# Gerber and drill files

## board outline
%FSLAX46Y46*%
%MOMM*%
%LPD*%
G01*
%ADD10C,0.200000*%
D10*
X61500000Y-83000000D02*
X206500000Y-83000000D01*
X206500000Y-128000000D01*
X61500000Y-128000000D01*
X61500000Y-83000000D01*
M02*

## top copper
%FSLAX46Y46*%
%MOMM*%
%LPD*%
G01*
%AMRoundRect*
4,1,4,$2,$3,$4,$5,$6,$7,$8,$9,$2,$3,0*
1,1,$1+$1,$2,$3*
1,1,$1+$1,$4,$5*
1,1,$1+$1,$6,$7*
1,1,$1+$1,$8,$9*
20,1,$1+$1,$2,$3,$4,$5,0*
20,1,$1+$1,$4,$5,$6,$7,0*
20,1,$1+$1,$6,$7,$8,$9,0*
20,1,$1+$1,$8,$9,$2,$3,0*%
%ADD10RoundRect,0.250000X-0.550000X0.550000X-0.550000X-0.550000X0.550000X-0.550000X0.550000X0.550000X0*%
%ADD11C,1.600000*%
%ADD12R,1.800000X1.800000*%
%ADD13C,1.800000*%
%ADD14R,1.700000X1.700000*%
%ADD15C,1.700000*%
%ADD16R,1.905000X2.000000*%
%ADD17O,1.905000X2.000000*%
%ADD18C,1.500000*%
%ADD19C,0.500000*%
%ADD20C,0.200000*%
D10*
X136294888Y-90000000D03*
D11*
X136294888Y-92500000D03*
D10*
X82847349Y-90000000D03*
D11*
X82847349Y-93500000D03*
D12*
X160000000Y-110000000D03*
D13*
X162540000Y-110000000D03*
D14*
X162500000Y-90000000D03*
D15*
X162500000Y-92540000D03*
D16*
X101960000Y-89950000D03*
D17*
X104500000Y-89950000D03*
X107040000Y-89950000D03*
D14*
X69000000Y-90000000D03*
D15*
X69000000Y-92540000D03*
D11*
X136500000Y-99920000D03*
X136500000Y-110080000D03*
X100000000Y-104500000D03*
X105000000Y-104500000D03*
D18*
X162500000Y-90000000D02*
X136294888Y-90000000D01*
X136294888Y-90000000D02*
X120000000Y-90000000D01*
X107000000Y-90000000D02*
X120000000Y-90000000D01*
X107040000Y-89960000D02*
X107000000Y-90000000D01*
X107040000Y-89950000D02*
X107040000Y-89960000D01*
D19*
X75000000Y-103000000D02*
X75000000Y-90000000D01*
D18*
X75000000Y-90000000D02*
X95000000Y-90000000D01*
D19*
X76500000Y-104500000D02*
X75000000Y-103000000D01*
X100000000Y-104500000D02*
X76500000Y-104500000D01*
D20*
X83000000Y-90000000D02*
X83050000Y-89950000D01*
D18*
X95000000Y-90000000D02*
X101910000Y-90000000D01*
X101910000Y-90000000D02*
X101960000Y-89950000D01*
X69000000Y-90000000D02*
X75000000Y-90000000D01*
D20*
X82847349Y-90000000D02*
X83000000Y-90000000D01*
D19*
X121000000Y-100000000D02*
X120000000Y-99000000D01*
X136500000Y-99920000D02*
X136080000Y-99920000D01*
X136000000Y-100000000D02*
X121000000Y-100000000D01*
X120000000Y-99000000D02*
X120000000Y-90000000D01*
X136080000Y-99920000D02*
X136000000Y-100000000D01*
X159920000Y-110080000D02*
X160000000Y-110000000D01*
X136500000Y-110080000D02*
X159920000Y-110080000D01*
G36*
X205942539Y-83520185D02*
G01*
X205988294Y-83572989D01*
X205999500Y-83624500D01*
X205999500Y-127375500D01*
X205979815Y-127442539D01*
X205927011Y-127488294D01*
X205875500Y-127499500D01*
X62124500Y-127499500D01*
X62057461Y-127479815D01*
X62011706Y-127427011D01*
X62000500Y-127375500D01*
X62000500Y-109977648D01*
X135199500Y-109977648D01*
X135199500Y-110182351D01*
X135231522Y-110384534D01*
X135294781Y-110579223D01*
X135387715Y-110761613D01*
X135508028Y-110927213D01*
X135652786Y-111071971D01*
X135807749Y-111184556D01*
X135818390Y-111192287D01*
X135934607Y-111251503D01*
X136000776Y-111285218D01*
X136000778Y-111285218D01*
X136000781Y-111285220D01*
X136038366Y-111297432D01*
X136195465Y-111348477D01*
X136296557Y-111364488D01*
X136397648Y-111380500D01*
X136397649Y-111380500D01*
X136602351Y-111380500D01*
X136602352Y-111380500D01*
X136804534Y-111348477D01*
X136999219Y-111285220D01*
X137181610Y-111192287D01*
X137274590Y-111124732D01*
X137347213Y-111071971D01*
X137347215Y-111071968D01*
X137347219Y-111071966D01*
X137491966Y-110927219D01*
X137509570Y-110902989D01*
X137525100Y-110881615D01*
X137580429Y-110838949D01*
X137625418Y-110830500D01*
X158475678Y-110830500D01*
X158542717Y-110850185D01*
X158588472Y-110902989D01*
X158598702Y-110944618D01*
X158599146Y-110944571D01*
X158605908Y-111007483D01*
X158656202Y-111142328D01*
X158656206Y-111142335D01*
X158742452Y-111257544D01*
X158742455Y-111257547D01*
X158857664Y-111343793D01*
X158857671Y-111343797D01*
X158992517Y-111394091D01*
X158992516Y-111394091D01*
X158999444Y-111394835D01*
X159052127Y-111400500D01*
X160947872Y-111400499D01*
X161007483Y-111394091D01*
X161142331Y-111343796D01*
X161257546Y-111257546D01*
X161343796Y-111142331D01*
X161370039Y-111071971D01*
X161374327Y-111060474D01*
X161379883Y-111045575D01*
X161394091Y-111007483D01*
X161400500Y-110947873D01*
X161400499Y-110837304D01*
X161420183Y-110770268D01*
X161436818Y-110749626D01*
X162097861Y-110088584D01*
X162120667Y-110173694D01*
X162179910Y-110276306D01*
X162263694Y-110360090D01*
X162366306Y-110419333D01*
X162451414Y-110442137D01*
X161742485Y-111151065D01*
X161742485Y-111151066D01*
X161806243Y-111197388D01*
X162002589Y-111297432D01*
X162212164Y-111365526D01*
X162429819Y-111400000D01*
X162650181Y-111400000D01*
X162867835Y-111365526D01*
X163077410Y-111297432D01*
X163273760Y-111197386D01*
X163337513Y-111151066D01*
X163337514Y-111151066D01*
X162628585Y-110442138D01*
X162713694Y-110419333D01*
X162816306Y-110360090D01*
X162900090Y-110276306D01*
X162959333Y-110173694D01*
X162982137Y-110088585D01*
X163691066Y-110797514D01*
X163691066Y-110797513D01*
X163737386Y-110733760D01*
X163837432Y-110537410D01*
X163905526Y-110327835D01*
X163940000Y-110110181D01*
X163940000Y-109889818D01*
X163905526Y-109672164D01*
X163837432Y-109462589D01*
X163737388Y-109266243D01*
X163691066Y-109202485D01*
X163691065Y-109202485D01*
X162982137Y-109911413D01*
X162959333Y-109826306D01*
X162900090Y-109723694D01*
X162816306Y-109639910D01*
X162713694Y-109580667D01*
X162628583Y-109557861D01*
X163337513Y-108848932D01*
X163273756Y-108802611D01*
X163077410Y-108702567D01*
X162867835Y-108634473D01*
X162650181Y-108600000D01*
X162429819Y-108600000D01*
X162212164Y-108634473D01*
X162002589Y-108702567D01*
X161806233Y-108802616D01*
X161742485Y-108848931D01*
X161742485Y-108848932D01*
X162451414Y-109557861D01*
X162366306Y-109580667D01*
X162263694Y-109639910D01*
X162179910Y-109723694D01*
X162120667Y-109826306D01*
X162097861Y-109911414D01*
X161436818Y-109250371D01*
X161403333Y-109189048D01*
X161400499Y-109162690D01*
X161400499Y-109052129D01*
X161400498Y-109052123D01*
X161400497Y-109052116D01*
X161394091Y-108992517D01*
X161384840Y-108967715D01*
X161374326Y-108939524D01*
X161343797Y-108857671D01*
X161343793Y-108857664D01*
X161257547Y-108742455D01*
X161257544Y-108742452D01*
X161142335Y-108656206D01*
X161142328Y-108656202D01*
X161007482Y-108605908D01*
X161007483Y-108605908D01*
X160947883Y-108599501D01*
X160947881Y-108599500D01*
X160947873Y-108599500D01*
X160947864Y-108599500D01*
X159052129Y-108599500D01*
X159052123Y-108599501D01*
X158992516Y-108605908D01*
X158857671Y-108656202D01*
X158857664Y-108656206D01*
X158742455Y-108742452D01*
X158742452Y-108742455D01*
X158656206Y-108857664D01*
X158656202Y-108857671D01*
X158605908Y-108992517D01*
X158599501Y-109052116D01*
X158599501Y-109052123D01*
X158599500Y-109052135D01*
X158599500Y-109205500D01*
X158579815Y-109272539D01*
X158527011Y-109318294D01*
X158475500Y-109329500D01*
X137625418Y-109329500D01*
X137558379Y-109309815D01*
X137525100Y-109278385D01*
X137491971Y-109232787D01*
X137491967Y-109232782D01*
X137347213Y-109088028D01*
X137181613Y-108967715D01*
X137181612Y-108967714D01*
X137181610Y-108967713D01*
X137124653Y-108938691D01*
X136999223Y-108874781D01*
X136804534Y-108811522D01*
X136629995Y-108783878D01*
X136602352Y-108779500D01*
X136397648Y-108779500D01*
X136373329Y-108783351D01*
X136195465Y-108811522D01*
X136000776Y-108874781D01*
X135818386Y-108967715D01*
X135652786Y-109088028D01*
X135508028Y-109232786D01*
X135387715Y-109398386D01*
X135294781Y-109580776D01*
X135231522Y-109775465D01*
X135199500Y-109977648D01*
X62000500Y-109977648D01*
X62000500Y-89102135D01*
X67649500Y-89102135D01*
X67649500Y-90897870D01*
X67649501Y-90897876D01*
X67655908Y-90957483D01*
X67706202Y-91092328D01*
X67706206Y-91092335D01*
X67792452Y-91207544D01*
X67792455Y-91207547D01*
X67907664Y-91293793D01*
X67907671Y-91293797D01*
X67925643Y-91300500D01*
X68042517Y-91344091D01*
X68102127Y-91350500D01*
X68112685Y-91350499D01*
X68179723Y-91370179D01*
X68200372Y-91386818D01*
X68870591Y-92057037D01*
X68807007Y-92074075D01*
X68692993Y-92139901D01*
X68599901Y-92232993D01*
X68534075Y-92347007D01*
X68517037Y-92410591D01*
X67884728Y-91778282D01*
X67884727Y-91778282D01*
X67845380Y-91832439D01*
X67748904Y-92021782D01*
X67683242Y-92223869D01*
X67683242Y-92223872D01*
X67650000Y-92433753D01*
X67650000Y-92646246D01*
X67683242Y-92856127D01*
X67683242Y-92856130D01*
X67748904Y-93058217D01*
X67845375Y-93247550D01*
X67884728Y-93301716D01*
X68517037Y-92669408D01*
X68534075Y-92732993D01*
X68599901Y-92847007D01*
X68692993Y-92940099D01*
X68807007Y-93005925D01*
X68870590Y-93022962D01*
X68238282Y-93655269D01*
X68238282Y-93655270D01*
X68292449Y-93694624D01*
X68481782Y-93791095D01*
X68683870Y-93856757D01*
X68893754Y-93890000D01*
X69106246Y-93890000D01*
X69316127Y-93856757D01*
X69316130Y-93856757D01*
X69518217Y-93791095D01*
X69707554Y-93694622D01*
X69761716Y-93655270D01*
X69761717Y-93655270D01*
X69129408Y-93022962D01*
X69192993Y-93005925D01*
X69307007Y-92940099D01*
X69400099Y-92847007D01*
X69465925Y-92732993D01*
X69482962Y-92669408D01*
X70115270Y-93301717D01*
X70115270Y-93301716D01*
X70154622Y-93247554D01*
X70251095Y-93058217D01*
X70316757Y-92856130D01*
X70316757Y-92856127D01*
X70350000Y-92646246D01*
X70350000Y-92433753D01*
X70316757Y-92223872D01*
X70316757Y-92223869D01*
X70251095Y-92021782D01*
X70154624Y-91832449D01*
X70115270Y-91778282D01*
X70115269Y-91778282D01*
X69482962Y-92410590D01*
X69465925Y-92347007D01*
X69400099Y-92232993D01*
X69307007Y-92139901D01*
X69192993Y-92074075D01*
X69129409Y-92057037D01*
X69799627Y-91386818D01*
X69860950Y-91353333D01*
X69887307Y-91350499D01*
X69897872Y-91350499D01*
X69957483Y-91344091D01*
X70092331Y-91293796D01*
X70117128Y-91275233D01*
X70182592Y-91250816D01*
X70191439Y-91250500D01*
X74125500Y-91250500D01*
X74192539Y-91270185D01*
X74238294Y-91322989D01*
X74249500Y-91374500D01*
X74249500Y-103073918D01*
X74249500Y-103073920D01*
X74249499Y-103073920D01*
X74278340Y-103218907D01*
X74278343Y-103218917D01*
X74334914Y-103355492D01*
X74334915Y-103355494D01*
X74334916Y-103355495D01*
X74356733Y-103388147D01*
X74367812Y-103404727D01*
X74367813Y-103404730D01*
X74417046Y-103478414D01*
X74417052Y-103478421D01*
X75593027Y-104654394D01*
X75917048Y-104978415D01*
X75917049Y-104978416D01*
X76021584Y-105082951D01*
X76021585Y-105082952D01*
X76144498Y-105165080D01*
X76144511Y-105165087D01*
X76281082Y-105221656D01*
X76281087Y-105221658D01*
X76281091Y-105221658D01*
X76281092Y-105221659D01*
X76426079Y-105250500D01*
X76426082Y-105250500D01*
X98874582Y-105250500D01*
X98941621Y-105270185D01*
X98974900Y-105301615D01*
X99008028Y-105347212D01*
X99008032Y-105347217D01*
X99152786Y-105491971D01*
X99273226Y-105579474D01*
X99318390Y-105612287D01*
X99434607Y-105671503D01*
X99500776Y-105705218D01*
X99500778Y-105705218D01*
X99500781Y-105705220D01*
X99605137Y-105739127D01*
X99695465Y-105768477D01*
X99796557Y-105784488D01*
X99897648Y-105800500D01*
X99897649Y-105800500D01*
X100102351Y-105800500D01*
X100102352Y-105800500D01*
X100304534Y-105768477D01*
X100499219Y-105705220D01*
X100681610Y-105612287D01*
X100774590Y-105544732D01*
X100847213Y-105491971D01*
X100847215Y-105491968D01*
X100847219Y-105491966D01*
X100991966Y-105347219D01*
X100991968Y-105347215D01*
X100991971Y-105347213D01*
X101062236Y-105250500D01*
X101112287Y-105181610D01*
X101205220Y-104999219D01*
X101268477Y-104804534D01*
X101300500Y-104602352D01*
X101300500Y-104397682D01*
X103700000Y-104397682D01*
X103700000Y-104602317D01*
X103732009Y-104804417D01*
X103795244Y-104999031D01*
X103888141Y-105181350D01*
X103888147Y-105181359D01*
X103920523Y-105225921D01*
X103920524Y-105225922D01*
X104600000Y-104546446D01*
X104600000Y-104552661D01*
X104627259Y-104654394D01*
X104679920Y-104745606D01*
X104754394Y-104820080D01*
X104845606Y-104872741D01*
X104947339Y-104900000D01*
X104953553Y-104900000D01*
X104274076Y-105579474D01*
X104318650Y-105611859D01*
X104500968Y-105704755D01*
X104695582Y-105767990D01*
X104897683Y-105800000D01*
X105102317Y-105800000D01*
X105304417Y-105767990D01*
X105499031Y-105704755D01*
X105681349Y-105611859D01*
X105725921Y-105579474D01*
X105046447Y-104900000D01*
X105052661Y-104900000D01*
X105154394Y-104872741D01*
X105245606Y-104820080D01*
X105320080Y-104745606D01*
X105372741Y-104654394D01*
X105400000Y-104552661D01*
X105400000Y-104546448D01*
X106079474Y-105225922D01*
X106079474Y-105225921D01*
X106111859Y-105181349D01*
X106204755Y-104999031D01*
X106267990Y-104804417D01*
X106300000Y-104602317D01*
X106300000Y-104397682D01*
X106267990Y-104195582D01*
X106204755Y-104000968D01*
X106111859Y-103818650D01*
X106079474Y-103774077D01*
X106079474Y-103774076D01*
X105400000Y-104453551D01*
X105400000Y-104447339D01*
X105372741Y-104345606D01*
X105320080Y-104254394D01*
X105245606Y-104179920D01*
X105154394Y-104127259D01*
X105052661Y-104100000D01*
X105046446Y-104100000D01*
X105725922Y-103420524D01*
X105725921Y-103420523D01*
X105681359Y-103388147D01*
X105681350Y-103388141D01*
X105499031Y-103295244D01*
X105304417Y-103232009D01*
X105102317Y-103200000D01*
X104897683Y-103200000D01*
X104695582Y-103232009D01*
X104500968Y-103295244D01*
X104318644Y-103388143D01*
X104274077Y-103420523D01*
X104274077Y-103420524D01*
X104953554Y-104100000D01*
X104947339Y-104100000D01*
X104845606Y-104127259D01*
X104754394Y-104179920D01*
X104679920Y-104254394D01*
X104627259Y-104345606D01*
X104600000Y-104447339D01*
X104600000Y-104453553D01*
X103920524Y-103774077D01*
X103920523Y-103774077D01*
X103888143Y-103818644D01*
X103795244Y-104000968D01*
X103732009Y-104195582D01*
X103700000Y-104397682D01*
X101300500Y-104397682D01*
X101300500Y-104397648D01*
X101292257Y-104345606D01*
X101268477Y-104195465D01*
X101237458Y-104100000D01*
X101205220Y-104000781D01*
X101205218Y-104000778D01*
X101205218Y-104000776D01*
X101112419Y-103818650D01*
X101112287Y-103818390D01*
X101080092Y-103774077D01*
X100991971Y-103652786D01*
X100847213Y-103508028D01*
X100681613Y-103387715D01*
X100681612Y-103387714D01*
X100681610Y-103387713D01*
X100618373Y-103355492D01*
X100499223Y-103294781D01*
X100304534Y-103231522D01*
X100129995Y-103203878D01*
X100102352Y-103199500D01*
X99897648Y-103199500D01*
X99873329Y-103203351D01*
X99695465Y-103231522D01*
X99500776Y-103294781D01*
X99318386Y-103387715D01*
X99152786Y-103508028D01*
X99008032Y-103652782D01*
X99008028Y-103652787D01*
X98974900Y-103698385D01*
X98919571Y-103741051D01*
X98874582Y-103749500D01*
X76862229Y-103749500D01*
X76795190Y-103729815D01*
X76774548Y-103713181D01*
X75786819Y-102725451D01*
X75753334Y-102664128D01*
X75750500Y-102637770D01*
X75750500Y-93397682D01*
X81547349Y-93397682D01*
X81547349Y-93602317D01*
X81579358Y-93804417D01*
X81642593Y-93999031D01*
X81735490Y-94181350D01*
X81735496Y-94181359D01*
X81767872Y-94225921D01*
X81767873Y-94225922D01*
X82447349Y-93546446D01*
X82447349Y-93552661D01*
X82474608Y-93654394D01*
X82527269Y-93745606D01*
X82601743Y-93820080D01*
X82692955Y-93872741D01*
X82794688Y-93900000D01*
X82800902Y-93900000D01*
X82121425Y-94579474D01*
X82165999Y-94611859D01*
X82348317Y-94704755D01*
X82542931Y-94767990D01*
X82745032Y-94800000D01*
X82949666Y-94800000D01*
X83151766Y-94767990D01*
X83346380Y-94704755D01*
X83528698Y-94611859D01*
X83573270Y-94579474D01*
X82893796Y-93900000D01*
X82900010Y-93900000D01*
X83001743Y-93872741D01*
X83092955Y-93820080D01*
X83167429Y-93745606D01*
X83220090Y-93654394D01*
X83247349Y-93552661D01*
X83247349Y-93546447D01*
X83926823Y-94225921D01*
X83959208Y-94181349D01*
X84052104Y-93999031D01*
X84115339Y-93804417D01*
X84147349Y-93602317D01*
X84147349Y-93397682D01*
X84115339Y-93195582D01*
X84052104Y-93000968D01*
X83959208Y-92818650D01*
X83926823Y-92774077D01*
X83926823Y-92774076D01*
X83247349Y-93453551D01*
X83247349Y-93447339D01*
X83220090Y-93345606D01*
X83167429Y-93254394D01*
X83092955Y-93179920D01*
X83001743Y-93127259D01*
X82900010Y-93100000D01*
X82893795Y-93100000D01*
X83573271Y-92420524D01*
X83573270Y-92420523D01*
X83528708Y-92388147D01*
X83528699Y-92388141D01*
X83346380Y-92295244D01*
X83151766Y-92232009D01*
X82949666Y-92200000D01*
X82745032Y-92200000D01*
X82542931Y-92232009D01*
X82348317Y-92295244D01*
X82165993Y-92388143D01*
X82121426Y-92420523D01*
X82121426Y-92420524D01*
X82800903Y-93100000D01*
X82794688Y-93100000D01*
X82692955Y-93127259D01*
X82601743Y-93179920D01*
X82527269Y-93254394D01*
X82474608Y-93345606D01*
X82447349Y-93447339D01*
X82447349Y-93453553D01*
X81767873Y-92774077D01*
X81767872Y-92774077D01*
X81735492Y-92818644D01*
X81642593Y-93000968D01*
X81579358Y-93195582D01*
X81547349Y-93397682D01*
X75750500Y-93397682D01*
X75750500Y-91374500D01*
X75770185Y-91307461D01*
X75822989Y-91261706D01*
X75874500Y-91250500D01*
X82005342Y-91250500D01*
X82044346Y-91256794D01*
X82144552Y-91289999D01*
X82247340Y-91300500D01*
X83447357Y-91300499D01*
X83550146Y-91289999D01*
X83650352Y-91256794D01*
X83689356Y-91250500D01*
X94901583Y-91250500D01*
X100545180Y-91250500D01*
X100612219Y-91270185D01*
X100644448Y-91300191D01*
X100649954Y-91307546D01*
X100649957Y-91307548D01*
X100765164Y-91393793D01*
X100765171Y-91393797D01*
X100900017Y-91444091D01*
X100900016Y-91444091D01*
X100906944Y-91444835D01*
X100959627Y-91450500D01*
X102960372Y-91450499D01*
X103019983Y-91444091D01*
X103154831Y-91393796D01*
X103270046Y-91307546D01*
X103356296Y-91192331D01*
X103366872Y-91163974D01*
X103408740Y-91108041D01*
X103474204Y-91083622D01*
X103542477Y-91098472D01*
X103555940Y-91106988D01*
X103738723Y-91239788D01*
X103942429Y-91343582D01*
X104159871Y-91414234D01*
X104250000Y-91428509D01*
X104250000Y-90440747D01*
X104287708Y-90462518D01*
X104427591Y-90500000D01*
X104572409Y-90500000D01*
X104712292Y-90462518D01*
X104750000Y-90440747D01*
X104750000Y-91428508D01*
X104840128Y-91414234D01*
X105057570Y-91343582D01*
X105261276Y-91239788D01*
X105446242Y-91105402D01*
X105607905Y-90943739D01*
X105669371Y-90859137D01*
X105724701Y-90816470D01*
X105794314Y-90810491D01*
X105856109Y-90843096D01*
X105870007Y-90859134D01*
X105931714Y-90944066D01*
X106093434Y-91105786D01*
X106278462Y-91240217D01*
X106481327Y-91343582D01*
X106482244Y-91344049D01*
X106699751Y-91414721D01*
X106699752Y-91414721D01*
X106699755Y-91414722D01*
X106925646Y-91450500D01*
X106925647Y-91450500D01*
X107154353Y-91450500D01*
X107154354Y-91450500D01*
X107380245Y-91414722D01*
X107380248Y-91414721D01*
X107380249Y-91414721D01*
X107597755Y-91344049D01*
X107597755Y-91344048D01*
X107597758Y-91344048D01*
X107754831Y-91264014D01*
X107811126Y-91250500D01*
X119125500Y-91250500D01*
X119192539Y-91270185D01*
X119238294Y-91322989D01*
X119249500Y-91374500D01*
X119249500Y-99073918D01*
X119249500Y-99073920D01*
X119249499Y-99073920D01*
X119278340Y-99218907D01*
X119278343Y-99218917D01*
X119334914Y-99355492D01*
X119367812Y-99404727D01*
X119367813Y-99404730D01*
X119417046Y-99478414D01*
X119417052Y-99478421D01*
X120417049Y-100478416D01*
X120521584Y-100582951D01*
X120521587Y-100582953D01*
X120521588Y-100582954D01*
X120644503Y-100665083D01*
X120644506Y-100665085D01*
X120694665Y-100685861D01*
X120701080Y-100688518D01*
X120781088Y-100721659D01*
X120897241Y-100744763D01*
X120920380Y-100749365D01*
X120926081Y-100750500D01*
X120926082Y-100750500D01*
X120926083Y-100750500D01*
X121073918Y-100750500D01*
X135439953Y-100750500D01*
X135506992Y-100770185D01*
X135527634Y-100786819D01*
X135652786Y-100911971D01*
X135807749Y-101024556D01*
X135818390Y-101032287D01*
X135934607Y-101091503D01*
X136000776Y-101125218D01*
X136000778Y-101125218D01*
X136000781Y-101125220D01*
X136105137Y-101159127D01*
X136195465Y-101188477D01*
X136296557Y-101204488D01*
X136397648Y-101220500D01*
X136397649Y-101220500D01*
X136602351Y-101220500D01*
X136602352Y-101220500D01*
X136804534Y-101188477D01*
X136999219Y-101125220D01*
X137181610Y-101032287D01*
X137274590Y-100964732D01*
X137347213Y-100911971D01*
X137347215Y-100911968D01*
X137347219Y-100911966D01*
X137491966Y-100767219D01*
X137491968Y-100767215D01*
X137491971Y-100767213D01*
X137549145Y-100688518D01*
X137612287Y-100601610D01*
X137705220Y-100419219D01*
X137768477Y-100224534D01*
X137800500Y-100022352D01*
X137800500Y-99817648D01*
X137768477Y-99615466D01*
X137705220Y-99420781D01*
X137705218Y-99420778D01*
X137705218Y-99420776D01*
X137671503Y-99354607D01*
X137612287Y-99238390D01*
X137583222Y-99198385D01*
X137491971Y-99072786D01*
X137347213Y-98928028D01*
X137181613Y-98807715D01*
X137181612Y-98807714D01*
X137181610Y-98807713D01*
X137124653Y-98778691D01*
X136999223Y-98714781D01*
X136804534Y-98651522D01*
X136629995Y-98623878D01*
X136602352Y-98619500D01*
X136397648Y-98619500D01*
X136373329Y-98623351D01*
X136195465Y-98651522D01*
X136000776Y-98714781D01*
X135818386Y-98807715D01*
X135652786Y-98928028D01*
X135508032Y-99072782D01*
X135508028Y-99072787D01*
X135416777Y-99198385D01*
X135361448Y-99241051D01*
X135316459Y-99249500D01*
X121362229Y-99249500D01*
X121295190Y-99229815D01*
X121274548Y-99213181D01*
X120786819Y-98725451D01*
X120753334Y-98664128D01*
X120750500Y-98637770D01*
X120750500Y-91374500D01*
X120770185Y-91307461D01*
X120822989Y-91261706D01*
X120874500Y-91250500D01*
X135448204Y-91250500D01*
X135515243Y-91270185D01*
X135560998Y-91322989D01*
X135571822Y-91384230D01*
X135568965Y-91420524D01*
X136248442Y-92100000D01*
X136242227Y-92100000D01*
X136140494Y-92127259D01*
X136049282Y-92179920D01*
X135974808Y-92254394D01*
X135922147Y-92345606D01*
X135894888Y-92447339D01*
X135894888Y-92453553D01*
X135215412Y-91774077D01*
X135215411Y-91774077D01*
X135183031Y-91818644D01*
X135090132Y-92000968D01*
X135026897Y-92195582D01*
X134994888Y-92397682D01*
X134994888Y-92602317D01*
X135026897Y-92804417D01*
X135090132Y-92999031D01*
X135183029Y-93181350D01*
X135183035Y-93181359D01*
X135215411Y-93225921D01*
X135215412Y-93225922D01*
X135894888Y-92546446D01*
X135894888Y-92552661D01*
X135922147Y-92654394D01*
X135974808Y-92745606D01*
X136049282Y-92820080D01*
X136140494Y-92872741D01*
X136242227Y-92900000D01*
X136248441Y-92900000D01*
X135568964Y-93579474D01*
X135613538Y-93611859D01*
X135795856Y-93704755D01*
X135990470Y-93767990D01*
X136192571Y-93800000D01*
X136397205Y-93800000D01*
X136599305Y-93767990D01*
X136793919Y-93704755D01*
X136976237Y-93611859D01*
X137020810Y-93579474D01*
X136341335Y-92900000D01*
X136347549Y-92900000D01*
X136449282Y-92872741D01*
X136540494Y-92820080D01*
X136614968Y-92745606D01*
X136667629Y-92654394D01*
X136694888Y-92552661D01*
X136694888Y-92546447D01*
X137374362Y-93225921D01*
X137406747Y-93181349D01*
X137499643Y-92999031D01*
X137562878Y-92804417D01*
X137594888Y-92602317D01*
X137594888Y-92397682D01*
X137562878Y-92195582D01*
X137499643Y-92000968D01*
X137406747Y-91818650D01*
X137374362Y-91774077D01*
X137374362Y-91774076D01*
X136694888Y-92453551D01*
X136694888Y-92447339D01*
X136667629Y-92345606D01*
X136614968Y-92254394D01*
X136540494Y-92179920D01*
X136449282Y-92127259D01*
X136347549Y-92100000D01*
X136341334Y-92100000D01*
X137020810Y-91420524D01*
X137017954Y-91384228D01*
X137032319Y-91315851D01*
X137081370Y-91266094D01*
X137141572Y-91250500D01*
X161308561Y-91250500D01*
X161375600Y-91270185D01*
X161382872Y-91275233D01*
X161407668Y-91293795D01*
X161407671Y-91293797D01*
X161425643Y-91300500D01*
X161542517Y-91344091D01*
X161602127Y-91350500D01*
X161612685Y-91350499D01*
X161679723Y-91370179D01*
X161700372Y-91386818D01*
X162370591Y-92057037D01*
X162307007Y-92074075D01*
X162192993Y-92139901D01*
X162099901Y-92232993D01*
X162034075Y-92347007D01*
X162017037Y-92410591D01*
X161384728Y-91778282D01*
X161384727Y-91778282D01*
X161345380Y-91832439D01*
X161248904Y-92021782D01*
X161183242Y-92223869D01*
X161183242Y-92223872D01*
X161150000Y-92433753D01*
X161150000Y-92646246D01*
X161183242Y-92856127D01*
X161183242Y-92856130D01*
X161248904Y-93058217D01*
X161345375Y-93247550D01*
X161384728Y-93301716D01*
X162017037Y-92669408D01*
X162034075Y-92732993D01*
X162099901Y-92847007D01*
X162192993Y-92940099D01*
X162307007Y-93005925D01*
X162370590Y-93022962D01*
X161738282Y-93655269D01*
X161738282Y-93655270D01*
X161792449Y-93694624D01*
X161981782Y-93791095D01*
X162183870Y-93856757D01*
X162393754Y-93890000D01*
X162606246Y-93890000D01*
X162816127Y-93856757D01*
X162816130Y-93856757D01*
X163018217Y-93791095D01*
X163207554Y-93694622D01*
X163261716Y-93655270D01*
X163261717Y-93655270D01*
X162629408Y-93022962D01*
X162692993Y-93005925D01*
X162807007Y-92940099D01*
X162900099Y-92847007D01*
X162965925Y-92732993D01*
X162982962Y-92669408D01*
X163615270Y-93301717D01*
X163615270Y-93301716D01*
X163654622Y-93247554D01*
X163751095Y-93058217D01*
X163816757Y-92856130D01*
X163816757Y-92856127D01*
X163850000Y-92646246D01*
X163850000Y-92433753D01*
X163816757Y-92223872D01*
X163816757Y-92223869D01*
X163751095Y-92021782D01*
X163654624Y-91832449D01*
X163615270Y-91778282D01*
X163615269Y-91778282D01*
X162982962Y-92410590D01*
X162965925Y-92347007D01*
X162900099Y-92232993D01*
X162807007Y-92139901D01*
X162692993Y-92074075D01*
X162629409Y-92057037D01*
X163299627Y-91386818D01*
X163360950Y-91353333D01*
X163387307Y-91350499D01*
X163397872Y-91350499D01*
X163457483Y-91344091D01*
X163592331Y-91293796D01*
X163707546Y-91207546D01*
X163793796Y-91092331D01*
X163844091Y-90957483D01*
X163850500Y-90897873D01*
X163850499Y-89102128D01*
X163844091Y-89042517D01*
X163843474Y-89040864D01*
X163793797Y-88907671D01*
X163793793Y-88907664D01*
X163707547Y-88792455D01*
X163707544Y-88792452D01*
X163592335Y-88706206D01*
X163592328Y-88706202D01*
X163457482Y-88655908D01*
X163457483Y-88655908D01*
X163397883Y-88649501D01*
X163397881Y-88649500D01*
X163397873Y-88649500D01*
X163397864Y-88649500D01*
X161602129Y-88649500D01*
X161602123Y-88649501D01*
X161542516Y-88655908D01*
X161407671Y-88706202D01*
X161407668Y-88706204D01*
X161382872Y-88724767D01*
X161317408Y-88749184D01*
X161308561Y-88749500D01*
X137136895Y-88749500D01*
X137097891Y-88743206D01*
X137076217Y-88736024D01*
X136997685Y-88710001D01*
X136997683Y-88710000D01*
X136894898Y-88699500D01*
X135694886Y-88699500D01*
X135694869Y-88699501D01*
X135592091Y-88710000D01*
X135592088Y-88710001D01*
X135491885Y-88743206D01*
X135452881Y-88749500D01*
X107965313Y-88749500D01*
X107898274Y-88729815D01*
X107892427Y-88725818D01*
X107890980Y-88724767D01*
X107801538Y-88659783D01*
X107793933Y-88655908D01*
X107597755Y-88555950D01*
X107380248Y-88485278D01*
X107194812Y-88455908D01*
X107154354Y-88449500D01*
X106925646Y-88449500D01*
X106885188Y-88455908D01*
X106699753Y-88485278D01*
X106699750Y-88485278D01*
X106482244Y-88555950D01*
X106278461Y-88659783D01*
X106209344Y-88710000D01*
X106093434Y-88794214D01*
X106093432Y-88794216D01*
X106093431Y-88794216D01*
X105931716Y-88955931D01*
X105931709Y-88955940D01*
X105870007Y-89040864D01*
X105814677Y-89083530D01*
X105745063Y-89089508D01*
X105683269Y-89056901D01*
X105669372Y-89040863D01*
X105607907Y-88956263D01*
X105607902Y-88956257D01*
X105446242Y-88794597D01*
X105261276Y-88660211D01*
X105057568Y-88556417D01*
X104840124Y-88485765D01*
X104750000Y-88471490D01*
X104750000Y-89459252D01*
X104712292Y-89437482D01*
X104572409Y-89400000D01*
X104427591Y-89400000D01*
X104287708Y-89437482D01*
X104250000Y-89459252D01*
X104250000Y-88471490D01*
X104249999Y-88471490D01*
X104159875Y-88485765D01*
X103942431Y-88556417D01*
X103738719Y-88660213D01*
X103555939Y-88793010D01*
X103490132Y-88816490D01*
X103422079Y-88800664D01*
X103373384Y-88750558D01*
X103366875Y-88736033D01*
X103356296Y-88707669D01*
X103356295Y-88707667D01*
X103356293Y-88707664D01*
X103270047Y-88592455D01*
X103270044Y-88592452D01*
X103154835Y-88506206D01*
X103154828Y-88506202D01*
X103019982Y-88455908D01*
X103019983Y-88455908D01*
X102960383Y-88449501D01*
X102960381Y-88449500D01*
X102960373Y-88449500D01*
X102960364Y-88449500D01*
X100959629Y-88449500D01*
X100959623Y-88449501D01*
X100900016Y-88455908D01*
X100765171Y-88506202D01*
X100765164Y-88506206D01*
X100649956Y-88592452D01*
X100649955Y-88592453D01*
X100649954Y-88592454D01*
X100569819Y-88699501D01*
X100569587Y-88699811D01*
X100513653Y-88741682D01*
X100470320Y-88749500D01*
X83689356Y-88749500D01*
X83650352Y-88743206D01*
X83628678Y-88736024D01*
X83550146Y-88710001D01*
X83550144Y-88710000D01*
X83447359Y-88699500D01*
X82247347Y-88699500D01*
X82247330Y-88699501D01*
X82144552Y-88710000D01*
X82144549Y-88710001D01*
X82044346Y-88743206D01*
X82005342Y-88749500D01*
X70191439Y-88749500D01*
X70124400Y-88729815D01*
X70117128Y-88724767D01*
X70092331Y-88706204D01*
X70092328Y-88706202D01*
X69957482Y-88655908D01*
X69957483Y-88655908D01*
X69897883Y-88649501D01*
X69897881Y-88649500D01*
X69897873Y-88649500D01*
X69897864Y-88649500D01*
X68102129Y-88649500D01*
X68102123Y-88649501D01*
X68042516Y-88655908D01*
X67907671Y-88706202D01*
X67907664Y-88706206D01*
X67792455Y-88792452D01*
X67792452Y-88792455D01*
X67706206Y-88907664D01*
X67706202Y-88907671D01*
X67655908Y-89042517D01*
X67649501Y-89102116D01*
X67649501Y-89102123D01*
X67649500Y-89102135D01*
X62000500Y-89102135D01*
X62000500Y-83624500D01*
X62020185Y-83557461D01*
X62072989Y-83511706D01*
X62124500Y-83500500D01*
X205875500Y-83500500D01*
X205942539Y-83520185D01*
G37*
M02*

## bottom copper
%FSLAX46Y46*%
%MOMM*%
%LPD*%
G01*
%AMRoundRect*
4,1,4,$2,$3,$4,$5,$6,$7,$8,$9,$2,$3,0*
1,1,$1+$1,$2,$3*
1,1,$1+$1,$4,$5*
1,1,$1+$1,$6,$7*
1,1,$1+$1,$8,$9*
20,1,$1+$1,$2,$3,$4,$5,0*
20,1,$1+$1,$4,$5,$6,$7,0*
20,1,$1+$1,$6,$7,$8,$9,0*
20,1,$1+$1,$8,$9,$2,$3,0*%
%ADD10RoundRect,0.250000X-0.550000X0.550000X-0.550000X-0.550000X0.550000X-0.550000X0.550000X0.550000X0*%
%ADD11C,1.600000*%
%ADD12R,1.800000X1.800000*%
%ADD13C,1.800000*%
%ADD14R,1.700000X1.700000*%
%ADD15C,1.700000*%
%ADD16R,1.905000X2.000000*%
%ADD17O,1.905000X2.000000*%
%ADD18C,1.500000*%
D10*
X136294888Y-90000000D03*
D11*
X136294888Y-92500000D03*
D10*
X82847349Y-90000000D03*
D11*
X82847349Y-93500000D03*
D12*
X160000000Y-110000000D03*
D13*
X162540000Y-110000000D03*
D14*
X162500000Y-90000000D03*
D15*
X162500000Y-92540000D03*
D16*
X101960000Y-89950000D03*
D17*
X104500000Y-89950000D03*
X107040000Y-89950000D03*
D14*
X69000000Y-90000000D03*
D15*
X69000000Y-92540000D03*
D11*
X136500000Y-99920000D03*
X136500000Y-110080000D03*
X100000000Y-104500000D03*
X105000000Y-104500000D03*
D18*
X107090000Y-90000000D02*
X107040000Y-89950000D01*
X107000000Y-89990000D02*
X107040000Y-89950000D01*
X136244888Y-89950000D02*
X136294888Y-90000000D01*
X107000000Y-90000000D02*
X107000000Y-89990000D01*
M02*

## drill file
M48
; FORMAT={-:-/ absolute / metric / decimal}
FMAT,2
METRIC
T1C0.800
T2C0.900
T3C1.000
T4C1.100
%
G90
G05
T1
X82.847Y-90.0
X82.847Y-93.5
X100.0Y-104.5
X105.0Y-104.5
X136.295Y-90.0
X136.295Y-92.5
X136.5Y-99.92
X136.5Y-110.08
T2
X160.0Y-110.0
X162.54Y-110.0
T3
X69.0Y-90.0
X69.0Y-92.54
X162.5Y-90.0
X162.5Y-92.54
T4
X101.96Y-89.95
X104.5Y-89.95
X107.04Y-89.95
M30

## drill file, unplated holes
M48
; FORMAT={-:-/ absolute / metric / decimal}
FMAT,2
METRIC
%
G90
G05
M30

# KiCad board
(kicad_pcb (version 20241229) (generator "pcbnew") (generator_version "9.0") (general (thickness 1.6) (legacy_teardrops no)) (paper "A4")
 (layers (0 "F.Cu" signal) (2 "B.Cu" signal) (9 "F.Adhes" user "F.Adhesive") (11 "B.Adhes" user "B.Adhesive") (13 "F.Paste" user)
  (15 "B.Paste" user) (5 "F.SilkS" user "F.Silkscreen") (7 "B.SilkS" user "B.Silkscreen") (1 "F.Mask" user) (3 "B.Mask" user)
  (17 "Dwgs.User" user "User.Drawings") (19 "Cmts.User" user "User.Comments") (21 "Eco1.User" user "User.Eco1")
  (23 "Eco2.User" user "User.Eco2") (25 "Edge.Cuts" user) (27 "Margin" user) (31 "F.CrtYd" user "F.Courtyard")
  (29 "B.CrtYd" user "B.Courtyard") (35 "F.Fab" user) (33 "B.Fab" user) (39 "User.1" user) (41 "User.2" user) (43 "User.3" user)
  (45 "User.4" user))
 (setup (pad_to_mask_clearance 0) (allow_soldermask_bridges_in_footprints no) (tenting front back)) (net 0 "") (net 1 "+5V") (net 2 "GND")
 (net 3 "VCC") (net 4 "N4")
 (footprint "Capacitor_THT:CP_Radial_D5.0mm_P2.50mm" (layer "F.Cu") (at 136.294888 90 -90)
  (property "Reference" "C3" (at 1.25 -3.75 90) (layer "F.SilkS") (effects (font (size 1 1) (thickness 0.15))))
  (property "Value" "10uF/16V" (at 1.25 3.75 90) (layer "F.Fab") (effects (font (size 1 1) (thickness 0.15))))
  (pad "1" thru_hole roundrect (at 0 0 270) (size 1.6 1.6) (drill 0.8) (layers "*.Cu" "*.Mask") (remove_unused_layers no)
   (roundrect_rratio 0.15625) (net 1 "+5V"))
  (pad "2" thru_hole circle (at 2.5 0 270) (size 1.6 1.6) (drill 0.8) (layers "*.Cu" "*.Mask") (remove_unused_layers no) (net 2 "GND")))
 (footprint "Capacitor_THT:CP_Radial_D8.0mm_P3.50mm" (layer "F.Cu") (at 82.847349 90 -90)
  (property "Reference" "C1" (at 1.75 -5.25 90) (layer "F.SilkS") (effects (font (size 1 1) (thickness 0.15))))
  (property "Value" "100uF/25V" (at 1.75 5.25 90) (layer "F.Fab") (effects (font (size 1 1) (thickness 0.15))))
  (pad "1" thru_hole roundrect (at 0 0 270) (size 1.6 1.6) (drill 0.8) (layers "*.Cu" "*.Mask") (remove_unused_layers no)
   (roundrect_rratio 0.15625) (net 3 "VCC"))
  (pad "2" thru_hole circle (at 3.5 0 270) (size 1.6 1.6) (drill 0.8) (layers "*.Cu" "*.Mask") (remove_unused_layers no) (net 2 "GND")))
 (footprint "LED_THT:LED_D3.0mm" (layer "F.Cu") (at 160 110)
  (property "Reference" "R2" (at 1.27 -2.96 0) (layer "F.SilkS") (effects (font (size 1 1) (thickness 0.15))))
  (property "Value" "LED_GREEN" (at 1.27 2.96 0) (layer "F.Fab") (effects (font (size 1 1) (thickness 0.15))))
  (pad "1" thru_hole rect (at 0 0) (size 1.8 1.8) (drill 0.9) (layers "*.Cu" "*.Mask") (remove_unused_layers no) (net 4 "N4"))
  (pad "2" thru_hole circle (at 2.54 0) (size 1.8 1.8) (drill 0.9) (layers "*.Cu" "*.Mask") (remove_unused_layers no) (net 2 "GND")))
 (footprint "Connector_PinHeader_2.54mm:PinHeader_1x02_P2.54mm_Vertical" (layer "F.Cu") (at 162.5 90)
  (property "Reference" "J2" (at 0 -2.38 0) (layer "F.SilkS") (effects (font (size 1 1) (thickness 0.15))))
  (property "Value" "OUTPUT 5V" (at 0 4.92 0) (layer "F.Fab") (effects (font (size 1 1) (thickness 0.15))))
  (pad "1" thru_hole rect (at 0 0) (size 1.7 1.7) (drill 1) (layers "*.Cu" "*.Mask") (remove_unused_layers no) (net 1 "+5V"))
  (pad "2" thru_hole circle (at 0 2.54) (size 1.7 1.7) (drill 1) (layers "*.Cu" "*.Mask") (remove_unused_layers no) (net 2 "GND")))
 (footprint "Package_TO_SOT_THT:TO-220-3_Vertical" (layer "F.Cu") (at 101.96 89.95)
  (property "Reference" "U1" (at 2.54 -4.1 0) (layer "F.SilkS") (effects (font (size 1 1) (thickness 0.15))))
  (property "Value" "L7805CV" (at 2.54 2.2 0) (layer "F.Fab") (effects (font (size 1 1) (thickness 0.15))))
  (pad "1" thru_hole rect (at 0 0) (size 1.905 2) (drill 1.1) (layers "*.Cu" "*.Mask") (remove_unused_layers no) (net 3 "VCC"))
  (pad "2" thru_hole oval (at 2.54 0) (size 1.905 2) (drill 1.1) (layers "*.Cu" "*.Mask") (remove_unused_layers no) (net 2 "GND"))
  (pad "3" thru_hole oval (at 5.08 0) (size 1.905 2) (drill 1.1) (layers "*.Cu" "*.Mask") (remove_unused_layers no) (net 1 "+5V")))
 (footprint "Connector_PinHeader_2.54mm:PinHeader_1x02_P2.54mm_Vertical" (layer "F.Cu") (at 69 90)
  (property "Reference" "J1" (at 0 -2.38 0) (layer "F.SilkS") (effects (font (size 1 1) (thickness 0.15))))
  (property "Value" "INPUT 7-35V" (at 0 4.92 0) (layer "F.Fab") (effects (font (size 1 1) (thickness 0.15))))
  (pad "1" thru_hole rect (at 0 0) (size 1.7 1.7) (drill 1) (layers "*.Cu" "*.Mask") (remove_unused_layers no) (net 3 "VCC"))
  (pad "2" thru_hole circle (at 0 2.54) (size 1.7 1.7) (drill 1) (layers "*.Cu" "*.Mask") (remove_unused_layers no) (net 2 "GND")))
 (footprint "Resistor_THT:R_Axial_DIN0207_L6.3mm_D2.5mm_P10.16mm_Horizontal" (layer "F.Cu") (at 136.5 99.92 -90)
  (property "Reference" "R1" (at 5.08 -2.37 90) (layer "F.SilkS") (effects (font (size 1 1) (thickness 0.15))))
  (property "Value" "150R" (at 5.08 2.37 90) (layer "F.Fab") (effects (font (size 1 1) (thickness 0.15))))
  (pad "1" thru_hole circle (at 0 0 270) (size 1.6 1.6) (drill 0.8) (layers "*.Cu" "*.Mask") (remove_unused_layers no) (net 1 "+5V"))
  (pad "2" thru_hole circle (at 10.16 0 270) (size 1.6 1.6) (drill 0.8) (layers "*.Cu" "*.Mask") (remove_unused_layers no) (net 4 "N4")))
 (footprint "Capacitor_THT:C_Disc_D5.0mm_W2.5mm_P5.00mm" (layer "F.Cu") (at 100 104.5)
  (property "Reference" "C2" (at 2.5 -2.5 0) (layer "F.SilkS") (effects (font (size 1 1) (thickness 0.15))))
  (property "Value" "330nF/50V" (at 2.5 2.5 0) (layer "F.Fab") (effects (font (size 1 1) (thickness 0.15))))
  (pad "1" thru_hole circle (at 0 0) (size 1.6 1.6) (drill 0.8) (layers "*.Cu" "*.Mask") (remove_unused_layers no) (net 3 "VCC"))
  (pad "2" thru_hole circle (at 5 0) (size 1.6 1.6) (drill 0.8) (layers "*.Cu" "*.Mask") (remove_unused_layers no) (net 2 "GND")))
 (gr_rect (start 61.5 83) (end 206.5 128) (stroke (width 0.2) (type solid)) (fill no) (layer "Edge.Cuts"))
 (segment (start 83 90) (end 83.05 89.95) (width 0.2) (layer "F.Cu") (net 3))
 (segment (start 75 103) (end 75 90) (width 0.5) (layer "F.Cu") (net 3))
 (segment (start 95 90) (end 101.91 90) (width 1.5) (layer "F.Cu") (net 3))
 (segment (start 101.91 90) (end 101.96 89.95) (width 1.5) (layer "F.Cu") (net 3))
 (segment (start 69 90) (end 75 90) (width 1.5) (layer "F.Cu") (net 3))
 (segment (start 76.5 104.5) (end 75 103) (width 0.5) (layer "F.Cu") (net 3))
 (segment (start 82.847349 90) (end 83 90) (width 0.2) (layer "F.Cu") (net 3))
 (segment (start 75 90) (end 95 90) (width 1.5) (layer "F.Cu") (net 3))
 (segment (start 100 104.5) (end 76.5 104.5) (width 0.5) (layer "F.Cu") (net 3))
 (segment (start 121 100) (end 120 99) (width 0.5) (layer "F.Cu") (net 1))
 (segment (start 107 90) (end 120 90) (width 1.5) (layer "F.Cu") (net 1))
 (segment (start 107.04 89.95) (end 107.04 89.96) (width 1.5) (layer "F.Cu") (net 1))
 (segment (start 107.04 89.96) (end 107 90) (width 1.5) (layer "F.Cu") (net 1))
 (segment (start 136.5 99.92) (end 136.08 99.92) (width 0.5) (layer "F.Cu") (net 1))
 (segment (start 136 100) (end 121 100) (width 0.5) (layer "F.Cu") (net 1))
 (segment (start 162.5 90) (end 136.294888 90) (width 1.5) (layer "F.Cu") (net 1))
 (segment (start 120 99) (end 120 90) (width 0.5) (layer "F.Cu") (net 1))
 (segment (start 136.08 99.92) (end 136 100) (width 0.5) (layer "F.Cu") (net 1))
 (segment (start 136.294888 90) (end 120 90) (width 1.5) (layer "F.Cu") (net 1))
 (segment (start 107.09 90) (end 107.04 89.95) (width 1.5) (layer "B.Cu") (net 1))
 (segment (start 107 89.99) (end 107.04 89.95) (width 1.5) (layer "B.Cu") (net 1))
 (segment (start 136.244888 89.95) (end 136.294888 90) (width 1.5) (layer "B.Cu") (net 1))
 (segment (start 107 90) (end 107 89.99) (width 1.5) (layer "B.Cu") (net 1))
 (segment (start 136.5 110.08) (end 159.92 110.08) (width 0.5) (layer "F.Cu") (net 4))
 (segment (start 159.92 110.08) (end 160 110) (width 0.5) (layer "F.Cu") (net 4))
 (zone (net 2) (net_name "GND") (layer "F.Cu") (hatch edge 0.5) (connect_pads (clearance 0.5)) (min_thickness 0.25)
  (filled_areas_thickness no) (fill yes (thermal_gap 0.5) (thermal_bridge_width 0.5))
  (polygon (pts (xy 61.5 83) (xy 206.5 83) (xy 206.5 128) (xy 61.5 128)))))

